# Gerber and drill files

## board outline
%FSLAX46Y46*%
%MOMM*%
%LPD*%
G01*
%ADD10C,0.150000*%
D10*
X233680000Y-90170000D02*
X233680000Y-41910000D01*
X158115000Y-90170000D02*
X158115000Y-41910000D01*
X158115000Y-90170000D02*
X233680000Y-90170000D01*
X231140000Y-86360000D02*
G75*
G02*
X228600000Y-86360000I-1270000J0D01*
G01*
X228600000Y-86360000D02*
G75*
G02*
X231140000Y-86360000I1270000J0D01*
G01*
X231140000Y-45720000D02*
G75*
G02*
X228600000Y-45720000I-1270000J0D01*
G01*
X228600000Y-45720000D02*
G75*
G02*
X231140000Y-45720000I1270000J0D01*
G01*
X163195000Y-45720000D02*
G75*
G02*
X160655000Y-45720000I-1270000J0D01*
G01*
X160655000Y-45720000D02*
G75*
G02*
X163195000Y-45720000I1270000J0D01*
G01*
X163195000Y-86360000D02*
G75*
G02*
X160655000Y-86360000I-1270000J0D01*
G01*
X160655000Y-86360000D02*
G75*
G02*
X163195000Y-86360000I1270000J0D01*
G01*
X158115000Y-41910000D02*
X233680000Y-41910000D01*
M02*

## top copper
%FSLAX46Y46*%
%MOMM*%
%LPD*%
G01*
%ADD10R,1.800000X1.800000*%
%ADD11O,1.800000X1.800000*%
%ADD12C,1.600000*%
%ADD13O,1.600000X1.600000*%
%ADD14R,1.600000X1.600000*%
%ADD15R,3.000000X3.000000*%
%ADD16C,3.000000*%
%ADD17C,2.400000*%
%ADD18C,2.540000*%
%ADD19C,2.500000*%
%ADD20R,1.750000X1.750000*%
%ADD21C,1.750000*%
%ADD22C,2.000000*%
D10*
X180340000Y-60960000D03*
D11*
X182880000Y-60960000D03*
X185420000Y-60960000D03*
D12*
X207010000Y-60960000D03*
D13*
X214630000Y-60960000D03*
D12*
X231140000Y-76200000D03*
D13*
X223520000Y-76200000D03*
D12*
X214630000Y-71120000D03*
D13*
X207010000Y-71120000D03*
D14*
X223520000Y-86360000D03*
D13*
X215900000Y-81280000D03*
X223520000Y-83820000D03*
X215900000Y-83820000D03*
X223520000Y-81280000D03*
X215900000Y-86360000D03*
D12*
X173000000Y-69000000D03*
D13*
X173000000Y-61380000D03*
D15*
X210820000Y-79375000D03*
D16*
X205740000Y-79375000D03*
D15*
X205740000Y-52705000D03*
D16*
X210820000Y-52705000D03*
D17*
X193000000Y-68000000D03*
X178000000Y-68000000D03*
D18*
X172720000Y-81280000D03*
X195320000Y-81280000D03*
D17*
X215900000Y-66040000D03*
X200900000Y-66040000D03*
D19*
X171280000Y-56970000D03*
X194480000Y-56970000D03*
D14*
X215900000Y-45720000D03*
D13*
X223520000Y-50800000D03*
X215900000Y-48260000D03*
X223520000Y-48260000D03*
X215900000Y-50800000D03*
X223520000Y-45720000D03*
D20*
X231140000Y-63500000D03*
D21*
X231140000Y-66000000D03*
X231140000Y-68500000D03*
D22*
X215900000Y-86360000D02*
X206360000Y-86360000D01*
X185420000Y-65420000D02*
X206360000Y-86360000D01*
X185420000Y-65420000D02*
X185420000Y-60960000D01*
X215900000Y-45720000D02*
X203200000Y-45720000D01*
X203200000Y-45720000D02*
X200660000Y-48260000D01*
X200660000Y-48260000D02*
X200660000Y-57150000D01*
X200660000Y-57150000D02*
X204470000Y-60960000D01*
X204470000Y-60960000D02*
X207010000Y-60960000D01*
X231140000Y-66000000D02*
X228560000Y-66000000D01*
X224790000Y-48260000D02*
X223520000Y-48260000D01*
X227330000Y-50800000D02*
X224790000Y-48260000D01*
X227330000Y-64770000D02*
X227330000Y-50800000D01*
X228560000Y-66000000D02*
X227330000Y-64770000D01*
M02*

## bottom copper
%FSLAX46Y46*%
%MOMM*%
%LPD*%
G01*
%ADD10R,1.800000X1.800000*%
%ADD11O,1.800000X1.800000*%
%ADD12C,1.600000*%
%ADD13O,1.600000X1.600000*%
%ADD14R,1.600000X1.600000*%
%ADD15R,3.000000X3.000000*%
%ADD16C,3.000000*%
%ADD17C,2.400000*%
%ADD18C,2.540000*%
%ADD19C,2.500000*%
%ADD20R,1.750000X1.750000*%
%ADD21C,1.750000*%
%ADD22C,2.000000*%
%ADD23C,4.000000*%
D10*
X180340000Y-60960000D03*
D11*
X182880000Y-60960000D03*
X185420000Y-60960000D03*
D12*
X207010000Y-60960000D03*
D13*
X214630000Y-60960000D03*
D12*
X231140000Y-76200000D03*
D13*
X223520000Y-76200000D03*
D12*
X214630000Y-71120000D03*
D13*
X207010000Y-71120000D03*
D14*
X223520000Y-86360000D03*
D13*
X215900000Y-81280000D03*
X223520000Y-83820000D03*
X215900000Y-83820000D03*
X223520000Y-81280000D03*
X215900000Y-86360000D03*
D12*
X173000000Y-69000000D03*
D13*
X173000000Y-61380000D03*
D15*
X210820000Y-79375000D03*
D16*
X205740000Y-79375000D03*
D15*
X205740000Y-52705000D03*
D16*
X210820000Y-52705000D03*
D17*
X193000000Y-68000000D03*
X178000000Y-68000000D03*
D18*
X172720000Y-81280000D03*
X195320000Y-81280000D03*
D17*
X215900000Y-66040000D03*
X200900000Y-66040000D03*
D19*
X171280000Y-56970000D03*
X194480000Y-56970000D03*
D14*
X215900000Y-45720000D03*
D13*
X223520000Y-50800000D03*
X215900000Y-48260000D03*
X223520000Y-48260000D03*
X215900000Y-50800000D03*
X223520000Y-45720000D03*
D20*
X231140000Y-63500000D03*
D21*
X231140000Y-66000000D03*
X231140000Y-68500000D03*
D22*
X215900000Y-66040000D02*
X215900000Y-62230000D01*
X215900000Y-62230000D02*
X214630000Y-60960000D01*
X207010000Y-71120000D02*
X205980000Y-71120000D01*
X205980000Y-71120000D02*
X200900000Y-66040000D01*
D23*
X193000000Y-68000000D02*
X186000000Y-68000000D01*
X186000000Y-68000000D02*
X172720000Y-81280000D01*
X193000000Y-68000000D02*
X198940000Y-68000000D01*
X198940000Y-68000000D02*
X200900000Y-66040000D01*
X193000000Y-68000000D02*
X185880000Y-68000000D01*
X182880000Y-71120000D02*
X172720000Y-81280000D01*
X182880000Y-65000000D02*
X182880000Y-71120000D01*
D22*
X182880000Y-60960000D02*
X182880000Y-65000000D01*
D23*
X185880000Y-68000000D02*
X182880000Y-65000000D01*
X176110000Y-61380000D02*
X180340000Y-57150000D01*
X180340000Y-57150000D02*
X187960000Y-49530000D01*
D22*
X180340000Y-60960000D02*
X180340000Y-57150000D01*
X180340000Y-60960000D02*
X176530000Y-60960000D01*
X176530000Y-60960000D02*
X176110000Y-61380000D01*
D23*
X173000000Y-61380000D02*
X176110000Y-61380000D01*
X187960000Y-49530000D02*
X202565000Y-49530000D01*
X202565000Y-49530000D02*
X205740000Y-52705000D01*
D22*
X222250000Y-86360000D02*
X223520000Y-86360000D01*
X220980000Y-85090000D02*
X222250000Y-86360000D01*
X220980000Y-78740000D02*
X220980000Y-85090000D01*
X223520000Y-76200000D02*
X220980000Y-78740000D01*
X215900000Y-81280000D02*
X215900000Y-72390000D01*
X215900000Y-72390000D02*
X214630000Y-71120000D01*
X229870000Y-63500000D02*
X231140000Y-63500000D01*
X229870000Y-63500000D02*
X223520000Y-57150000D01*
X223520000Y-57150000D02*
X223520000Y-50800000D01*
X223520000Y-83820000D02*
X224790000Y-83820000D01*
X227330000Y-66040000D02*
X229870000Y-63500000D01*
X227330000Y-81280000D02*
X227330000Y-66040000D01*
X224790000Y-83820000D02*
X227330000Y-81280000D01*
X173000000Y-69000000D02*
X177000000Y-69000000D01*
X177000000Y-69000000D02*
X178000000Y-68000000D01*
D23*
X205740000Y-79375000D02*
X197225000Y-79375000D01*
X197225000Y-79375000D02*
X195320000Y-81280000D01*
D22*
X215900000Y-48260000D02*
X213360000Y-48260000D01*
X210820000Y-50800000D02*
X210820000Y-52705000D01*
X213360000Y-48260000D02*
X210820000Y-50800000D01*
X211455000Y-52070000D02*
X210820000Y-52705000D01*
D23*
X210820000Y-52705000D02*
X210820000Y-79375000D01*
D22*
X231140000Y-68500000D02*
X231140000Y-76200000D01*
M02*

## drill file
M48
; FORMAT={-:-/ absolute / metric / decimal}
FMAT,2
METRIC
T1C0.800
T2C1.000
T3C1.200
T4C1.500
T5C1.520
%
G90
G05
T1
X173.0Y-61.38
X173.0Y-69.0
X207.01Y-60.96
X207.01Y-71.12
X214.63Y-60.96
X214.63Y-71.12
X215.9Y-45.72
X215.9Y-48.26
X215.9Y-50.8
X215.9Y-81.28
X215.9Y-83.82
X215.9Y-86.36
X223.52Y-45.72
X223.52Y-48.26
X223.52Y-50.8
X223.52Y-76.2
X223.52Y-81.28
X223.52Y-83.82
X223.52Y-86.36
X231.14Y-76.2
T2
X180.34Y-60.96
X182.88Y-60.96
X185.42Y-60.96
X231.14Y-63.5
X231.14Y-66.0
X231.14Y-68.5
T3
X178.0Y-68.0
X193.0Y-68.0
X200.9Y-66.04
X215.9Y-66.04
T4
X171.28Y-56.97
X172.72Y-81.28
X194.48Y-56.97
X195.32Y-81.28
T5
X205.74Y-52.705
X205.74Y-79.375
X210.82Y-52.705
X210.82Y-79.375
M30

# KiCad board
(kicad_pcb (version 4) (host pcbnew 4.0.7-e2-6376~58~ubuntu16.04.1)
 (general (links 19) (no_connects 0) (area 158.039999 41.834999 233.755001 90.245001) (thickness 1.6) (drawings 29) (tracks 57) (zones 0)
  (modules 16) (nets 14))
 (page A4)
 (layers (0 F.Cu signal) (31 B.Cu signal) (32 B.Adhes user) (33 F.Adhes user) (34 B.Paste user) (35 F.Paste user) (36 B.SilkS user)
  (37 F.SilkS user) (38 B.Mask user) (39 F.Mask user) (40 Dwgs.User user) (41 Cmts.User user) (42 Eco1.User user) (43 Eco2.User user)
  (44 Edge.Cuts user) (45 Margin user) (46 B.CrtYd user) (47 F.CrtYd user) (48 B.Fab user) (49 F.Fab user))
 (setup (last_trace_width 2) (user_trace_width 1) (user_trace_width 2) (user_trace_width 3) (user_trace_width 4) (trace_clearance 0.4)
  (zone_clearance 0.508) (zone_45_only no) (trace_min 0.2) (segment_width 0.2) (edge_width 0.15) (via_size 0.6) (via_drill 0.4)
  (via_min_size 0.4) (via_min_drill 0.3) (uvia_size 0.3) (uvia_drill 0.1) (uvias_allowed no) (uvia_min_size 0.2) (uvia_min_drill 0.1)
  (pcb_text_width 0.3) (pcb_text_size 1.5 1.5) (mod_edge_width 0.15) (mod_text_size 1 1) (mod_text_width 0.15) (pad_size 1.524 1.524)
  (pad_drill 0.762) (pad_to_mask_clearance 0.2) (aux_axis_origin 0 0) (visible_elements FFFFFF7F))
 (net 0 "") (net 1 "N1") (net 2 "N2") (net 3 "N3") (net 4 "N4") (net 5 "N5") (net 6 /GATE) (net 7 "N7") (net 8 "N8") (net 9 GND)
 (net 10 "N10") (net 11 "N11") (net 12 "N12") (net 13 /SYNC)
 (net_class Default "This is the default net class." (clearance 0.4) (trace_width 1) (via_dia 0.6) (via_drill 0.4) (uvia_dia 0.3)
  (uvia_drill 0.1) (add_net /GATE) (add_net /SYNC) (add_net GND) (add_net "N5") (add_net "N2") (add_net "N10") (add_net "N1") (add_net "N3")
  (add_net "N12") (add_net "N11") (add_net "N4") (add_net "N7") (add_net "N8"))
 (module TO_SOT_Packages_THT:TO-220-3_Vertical (layer F.Cu) (at 180.34 60.96)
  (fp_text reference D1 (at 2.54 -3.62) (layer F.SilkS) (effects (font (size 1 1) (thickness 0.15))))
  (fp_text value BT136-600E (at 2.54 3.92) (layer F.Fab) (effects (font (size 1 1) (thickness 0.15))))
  (pad 1 thru_hole rect (at 0 0) (size 1.8 1.8) (drill 1) (layers *.Cu *.Mask) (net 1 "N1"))
  (pad 2 thru_hole oval (at 2.54 0) (size 1.8 1.8) (drill 1) (layers *.Cu *.Mask) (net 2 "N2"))
  (pad 3 thru_hole oval (at 5.08 0) (size 1.8 1.8) (drill 1) (layers *.Cu *.Mask) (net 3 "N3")))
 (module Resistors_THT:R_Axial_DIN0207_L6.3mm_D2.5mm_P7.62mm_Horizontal (layer F.Cu) (at 207.01 60.96)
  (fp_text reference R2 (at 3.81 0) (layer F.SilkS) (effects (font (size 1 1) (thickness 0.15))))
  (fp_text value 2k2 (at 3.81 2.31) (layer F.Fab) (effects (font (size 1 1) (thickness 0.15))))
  (pad 1 thru_hole circle (at 0 0) (size 1.6 1.6) (drill 0.8) (layers *.Cu *.Mask) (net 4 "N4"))
  (pad 2 thru_hole oval (at 7.62 0) (size 1.6 1.6) (drill 0.8) (layers *.Cu *.Mask) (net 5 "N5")))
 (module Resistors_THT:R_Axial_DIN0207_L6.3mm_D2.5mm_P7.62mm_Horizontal (layer F.Cu) (at 231.14 76.2 180)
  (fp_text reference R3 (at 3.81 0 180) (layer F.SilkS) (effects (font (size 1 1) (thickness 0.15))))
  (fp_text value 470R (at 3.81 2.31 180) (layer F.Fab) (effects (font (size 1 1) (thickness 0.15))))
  (pad 1 thru_hole circle (at 0 0 180) (size 1.6 1.6) (drill 0.8) (layers *.Cu *.Mask) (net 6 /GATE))
  (pad 2 thru_hole oval (at 7.62 0 180) (size 1.6 1.6) (drill 0.8) (layers *.Cu *.Mask) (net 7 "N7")))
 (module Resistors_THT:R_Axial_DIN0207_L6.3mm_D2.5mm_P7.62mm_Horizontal (layer F.Cu) (at 214.63 71.12 180)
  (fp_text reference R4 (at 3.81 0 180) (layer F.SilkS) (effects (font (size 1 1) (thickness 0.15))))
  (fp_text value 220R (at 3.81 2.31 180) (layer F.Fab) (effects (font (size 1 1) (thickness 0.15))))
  (pad 1 thru_hole circle (at 0 0 180) (size 1.6 1.6) (drill 0.8) (layers *.Cu *.Mask) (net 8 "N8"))
  (pad 2 thru_hole oval (at 7.62 0 180) (size 1.6 1.6) (drill 0.8) (layers *.Cu *.Mask) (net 2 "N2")))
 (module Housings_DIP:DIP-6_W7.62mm (layer F.Cu) (at 223.52 86.36 180)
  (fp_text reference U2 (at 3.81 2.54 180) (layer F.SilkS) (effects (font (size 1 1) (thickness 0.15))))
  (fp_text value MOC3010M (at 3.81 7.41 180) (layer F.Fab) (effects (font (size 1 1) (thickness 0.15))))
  (pad 1 thru_hole rect (at 0 0 180) (size 1.6 1.6) (drill 0.8) (layers *.Cu *.Mask) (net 7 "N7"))
  (pad 4 thru_hole oval (at 7.62 5.08 180) (size 1.6 1.6) (drill 0.8) (layers *.Cu *.Mask) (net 8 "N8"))
  (pad 2 thru_hole oval (at 0 2.54 180) (size 1.6 1.6) (drill 0.8) (layers *.Cu *.Mask) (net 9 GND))
  (pad 5 thru_hole oval (at 7.62 2.54 180) (size 1.6 1.6) (drill 0.8) (layers *.Cu *.Mask))
  (pad 3 thru_hole oval (at 0 5.08 180) (size 1.6 1.6) (drill 0.8) (layers *.Cu *.Mask))
  (pad 6 thru_hole oval (at 7.62 0 180) (size 1.6 1.6) (drill 0.8) (layers *.Cu *.Mask) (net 3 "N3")))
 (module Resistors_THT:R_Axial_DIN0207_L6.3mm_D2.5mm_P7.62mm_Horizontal (layer F.Cu) (at 173 69 90)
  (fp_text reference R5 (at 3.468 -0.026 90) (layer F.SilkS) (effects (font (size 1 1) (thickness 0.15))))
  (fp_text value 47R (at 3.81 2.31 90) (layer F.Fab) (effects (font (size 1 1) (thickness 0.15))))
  (pad 1 thru_hole circle (at 0 0 90) (size 1.6 1.6) (drill 0.8) (layers *.Cu *.Mask) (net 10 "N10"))
  (pad 2 thru_hole oval (at 7.62 0 90) (size 1.6 1.6) (drill 0.8) (layers *.Cu *.Mask) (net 1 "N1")))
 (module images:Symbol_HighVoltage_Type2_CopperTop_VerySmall (layer F.Cu) (at 163.83 74.93 270)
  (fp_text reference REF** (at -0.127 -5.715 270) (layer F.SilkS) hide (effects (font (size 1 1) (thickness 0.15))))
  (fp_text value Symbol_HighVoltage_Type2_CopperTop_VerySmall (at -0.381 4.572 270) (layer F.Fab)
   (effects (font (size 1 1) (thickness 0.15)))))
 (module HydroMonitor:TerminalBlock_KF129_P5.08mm (layer F.Cu) (at 210.82 79.375 180)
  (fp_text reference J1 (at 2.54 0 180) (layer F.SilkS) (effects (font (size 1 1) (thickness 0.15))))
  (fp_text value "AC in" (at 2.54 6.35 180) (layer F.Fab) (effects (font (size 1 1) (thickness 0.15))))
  (pad 1 thru_hole rect (at 0 0 180) (size 3 3) (drill 1.52) (layers *.Cu *.Mask) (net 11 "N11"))
  (pad 2 thru_hole circle (at 5.08 0 180) (size 3 3) (drill 1.52) (layers *.Cu *.Mask) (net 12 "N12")))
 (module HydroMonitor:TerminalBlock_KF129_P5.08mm (layer F.Cu) (at 205.74 52.705)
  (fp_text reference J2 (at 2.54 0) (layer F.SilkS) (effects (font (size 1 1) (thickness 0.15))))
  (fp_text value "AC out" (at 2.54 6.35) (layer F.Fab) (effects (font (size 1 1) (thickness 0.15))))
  (pad 1 thru_hole rect (at 0 0) (size 3 3) (drill 1.52) (layers *.Cu *.Mask) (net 1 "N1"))
  (pad 2 thru_hole circle (at 5.08 0) (size 3 3) (drill 1.52) (layers *.Cu *.Mask) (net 11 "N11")))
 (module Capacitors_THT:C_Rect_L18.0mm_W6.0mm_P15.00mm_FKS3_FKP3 (layer F.Cu) (at 193 68 180)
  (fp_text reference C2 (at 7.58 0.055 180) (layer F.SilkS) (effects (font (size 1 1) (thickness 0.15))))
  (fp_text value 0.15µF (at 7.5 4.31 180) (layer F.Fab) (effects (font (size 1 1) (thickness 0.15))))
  (pad 1 thru_hole circle (at 0 0 180) (size 2.4 2.4) (drill 1.2) (layers *.Cu *.Mask) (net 2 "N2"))
  (pad 2 thru_hole circle (at 15 0 180) (size 2.4 2.4) (drill 1.2) (layers *.Cu *.Mask) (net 10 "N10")))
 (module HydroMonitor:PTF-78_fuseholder (layer F.Cu) (at 172.72 81.28)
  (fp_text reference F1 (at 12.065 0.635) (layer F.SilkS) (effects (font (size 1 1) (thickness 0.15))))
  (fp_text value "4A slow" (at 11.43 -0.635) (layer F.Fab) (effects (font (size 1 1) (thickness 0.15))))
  (pad 1 thru_hole circle (at 0 0) (size 2.54 2.54) (drill 1.5) (layers *.Cu *.Mask) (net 2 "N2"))
  (pad 2 thru_hole circle (at 22.6 0) (size 2.54 2.54) (drill 1.5) (layers *.Cu *.Mask) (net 12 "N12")))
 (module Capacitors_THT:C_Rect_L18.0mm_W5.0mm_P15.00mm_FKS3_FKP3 (layer F.Cu) (at 215.9 66.04 180)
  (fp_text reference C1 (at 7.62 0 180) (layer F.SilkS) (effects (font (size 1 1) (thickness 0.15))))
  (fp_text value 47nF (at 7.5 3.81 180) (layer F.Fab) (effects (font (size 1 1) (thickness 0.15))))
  (pad 1 thru_hole circle (at 0 0 180) (size 2.4 2.4) (drill 1.2) (layers *.Cu *.Mask) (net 5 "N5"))
  (pad 2 thru_hole circle (at 15 0 180) (size 2.4 2.4) (drill 1.2) (layers *.Cu *.Mask) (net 2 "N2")))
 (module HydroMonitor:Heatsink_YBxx (layer F.Cu) (at 182.88 58.42 180)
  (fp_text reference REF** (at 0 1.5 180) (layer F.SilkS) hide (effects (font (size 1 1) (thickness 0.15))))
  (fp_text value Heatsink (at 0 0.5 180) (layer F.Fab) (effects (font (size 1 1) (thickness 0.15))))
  (pad "" thru_hole circle (at 11.6 1.45 180) (size 2.5 2.5) (drill 1.5) (layers *.Cu *.Mask))
  (pad "" thru_hole circle (at -11.6 1.45 180) (size 2.5 2.5) (drill 1.5) (layers *.Cu *.Mask)))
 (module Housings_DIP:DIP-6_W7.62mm (layer F.Cu) (at 215.9 45.72)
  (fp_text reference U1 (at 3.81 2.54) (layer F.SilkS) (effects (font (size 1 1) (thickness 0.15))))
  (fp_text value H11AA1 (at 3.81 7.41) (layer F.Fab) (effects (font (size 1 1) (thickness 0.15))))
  (pad 1 thru_hole rect (at 0 0) (size 1.6 1.6) (drill 0.8) (layers *.Cu *.Mask) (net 4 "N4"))
  (pad 4 thru_hole oval (at 7.62 5.08) (size 1.6 1.6) (drill 0.8) (layers *.Cu *.Mask) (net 9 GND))
  (pad 2 thru_hole oval (at 0 2.54) (size 1.6 1.6) (drill 0.8) (layers *.Cu *.Mask) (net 11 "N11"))
  (pad 5 thru_hole oval (at 7.62 2.54) (size 1.6 1.6) (drill 0.8) (layers *.Cu *.Mask) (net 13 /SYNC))
  (pad 3 thru_hole oval (at 0 5.08) (size 1.6 1.6) (drill 0.8) (layers *.Cu *.Mask))
  (pad 6 thru_hole oval (at 7.62 0) (size 1.6 1.6) (drill 0.8) (layers *.Cu *.Mask)))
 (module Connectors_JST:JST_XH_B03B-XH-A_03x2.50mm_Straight (layer F.Cu) (at 231.14 63.5 270)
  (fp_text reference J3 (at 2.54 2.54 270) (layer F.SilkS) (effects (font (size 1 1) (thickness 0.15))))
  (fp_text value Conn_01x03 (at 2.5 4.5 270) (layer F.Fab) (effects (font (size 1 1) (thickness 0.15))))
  (pad 1 thru_hole rect (at 0 0 270) (size 1.75 1.75) (drill 1) (layers *.Cu *.Mask) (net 9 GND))
  (pad 2 thru_hole circle (at 2.5 0 270) (size 1.75 1.75) (drill 1) (layers *.Cu *.Mask) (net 13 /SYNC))
  (pad 3 thru_hole circle (at 5 0 270) (size 1.75 1.75) (drill 1) (layers *.Cu *.Mask) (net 6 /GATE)))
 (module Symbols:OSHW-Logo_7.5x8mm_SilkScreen (layer F.Cu) (at 227.965 55.245 90)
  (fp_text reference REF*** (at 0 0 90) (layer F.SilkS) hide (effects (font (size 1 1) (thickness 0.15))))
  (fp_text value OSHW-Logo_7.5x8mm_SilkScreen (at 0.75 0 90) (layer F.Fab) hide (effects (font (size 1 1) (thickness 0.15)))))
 (gr_line (start 233.68 90.17) (end 233.68 41.91) (angle 90) (layer Edge.Cuts) (width 0.15))
 (gr_line (start 158.115 90.17) (end 158.115 41.91) (angle 90) (layer Edge.Cuts) (width 0.15))
 (gr_line (start 158.115 90.17) (end 233.68 90.17) (angle 90) (layer Edge.Cuts) (width 0.15))
 (gr_circle (center 229.87 86.36) (end 231.14 86.36) (layer Edge.Cuts) (width 0.15))
 (gr_circle (center 229.87 45.72) (end 231.14 45.72) (layer Edge.Cuts) (width 0.15))
 (gr_circle (center 161.925 45.72) (end 161.925 44.45) (layer Edge.Cuts) (width 0.15))
 (gr_circle (center 161.925 86.36) (end 161.925 87.63) (layer Edge.Cuts) (width 0.15))
 (gr_line (start 158.115 41.91) (end 233.68 41.91) (angle 90) (layer Edge.Cuts) (width 0.15))
 (segment (start 215.9 66.04) (end 215.9 62.23) (width 2) (layer B.Cu) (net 5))
 (segment (start 215.9 62.23) (end 214.63 60.96) (width 2) (layer B.Cu) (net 5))
 (segment (start 207.01 71.12) (end 205.98 71.12) (width 2) (layer B.Cu) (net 2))
 (segment (start 205.98 71.12) (end 200.9 66.04) (width 2) (layer B.Cu) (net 2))
 (segment (start 193 68) (end 186 68) (width 4) (layer B.Cu) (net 2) (status 10))
 (segment (start 186 68) (end 172.72 81.28) (width 4) (layer B.Cu) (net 2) (status 20))
 (segment (start 193 68) (end 198.94 68) (width 4) (layer B.Cu) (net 2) (status 10))
 (segment (start 198.94 68) (end 200.9 66.04) (width 4) (layer B.Cu) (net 2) (status 20))
 (segment (start 193 68) (end 185.88 68) (width 4) (layer B.Cu) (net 2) (status 10))
 (segment (start 182.88 71.12) (end 172.72 81.28) (width 4) (layer B.Cu) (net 2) (status 20))
 (segment (start 182.88 65) (end 182.88 71.12) (width 4) (layer B.Cu) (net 2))
 (segment (start 182.88 60.96) (end 182.88 65) (width 2) (layer B.Cu) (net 2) (status 10))
 (segment (start 185.88 68) (end 182.88 65) (width 4) (layer B.Cu) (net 2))
 (segment (start 176.11 61.38) (end 180.34 57.15) (width 4) (layer B.Cu) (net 1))
 (segment (start 180.34 57.15) (end 187.96 49.53) (width 4) (layer B.Cu) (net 1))
 (segment (start 180.34 60.96) (end 180.34 57.15) (width 2) (layer B.Cu) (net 1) (status 10))
 (segment (start 180.34 60.96) (end 176.53 60.96) (width 2) (layer B.Cu) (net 1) (status 10))
 (segment (start 176.53 60.96) (end 176.11 61.38) (width 2) (layer B.Cu) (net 1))
 (segment (start 173 61.38) (end 176.11 61.38) (width 4) (layer B.Cu) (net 1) (status 10))
 (segment (start 187.96 49.53) (end 202.565 49.53) (width 4) (layer B.Cu) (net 1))
 (segment (start 202.565 49.53) (end 205.74 52.705) (width 4) (layer B.Cu) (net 1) (status 20))
 (segment (start 215.9 86.36) (end 206.36 86.36) (width 2) (layer F.Cu) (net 3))
 (segment (start 185.42 65.42) (end 206.36 86.36) (width 2) (layer F.Cu) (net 3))
 (segment (start 185.42 65.42) (end 185.42 60.96) (width 2) (layer F.Cu) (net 3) (status 10))
 (segment (start 222.25 86.36) (end 223.52 86.36) (width 2) (layer B.Cu) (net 7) (status 20))
 (segment (start 220.98 85.09) (end 222.25 86.36) (width 2) (layer B.Cu) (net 7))
 (segment (start 220.98 78.74) (end 220.98 85.09) (width 2) (layer B.Cu) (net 7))
 (segment (start 223.52 76.2) (end 220.98 78.74) (width 2) (layer B.Cu) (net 7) (status 10))
 (segment (start 215.9 81.28) (end 215.9 72.39) (width 2) (layer B.Cu) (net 8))
 (segment (start 215.9 72.39) (end 214.63 71.12) (width 2) (layer B.Cu) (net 8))
 (segment (start 229.87 63.5) (end 231.14 63.5) (width 2) (layer B.Cu) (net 9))
 (segment (start 229.87 63.5) (end 223.52 57.15) (width 2) (layer B.Cu) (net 9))
 (segment (start 223.52 57.15) (end 223.52 50.8) (width 2) (layer B.Cu) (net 9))
 (segment (start 223.52 83.82) (end 224.79 83.82) (width 2) (layer B.Cu) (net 9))
 (segment (start 227.33 66.04) (end 229.87 63.5) (width 2) (layer B.Cu) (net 9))
 (segment (start 227.33 81.28) (end 227.33 66.04) (width 2) (layer B.Cu) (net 9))
 (segment (start 224.79 83.82) (end 227.33 81.28) (width 2) (layer B.Cu) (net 9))
 (segment (start 173 69) (end 177 69) (width 2) (layer B.Cu) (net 10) (status 10))
 (segment (start 177 69) (end 178 68) (width 2) (layer B.Cu) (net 10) (status 20))
 (segment (start 205.74 79.375) (end 197.225 79.375) (width 4) (layer B.Cu) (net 12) (status 10))
 (segment (start 197.225 79.375) (end 195.32 81.28) (width 4) (layer B.Cu) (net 12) (status 20))
 (segment (start 215.9 48.26) (end 213.36 48.26) (width 2) (layer B.Cu) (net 11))
 (segment (start 210.82 50.8) (end 210.82 52.705) (width 2) (layer B.Cu) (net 11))
 (segment (start 213.36 48.26) (end 210.82 50.8) (width 2) (layer B.Cu) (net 11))
 (segment (start 211.455 52.07) (end 210.82 52.705) (width 2) (layer B.Cu) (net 11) (status 30))
 (segment (start 210.82 52.705) (end 210.82 79.375) (width 4) (layer B.Cu) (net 11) (status 30))
 (segment (start 215.9 45.72) (end 203.2 45.72) (width 2) (layer F.Cu) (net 4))
 (segment (start 203.2 45.72) (end 200.66 48.26) (width 2) (layer F.Cu) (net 4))
 (segment (start 200.66 48.26) (end 200.66 57.15) (width 2) (layer F.Cu) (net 4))
 (segment (start 200.66 57.15) (end 204.47 60.96) (width 2) (layer F.Cu) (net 4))
 (segment (start 204.47 60.96) (end 207.01 60.96) (width 2) (layer F.Cu) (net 4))
 (segment (start 231.14 66) (end 228.56 66) (width 2) (layer F.Cu) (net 13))
 (segment (start 224.79 48.26) (end 223.52 48.26) (width 2) (layer F.Cu) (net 13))
 (segment (start 227.33 50.8) (end 224.79 48.26) (width 2) (layer F.Cu) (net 13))
 (segment (start 227.33 64.77) (end 227.33 50.8) (width 2) (layer F.Cu) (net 13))
 (segment (start 228.56 66) (end 227.33 64.77) (width 2) (layer F.Cu) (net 13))
 (segment (start 231.14 68.5) (end 231.14 76.2) (width 2) (layer B.Cu) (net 6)))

